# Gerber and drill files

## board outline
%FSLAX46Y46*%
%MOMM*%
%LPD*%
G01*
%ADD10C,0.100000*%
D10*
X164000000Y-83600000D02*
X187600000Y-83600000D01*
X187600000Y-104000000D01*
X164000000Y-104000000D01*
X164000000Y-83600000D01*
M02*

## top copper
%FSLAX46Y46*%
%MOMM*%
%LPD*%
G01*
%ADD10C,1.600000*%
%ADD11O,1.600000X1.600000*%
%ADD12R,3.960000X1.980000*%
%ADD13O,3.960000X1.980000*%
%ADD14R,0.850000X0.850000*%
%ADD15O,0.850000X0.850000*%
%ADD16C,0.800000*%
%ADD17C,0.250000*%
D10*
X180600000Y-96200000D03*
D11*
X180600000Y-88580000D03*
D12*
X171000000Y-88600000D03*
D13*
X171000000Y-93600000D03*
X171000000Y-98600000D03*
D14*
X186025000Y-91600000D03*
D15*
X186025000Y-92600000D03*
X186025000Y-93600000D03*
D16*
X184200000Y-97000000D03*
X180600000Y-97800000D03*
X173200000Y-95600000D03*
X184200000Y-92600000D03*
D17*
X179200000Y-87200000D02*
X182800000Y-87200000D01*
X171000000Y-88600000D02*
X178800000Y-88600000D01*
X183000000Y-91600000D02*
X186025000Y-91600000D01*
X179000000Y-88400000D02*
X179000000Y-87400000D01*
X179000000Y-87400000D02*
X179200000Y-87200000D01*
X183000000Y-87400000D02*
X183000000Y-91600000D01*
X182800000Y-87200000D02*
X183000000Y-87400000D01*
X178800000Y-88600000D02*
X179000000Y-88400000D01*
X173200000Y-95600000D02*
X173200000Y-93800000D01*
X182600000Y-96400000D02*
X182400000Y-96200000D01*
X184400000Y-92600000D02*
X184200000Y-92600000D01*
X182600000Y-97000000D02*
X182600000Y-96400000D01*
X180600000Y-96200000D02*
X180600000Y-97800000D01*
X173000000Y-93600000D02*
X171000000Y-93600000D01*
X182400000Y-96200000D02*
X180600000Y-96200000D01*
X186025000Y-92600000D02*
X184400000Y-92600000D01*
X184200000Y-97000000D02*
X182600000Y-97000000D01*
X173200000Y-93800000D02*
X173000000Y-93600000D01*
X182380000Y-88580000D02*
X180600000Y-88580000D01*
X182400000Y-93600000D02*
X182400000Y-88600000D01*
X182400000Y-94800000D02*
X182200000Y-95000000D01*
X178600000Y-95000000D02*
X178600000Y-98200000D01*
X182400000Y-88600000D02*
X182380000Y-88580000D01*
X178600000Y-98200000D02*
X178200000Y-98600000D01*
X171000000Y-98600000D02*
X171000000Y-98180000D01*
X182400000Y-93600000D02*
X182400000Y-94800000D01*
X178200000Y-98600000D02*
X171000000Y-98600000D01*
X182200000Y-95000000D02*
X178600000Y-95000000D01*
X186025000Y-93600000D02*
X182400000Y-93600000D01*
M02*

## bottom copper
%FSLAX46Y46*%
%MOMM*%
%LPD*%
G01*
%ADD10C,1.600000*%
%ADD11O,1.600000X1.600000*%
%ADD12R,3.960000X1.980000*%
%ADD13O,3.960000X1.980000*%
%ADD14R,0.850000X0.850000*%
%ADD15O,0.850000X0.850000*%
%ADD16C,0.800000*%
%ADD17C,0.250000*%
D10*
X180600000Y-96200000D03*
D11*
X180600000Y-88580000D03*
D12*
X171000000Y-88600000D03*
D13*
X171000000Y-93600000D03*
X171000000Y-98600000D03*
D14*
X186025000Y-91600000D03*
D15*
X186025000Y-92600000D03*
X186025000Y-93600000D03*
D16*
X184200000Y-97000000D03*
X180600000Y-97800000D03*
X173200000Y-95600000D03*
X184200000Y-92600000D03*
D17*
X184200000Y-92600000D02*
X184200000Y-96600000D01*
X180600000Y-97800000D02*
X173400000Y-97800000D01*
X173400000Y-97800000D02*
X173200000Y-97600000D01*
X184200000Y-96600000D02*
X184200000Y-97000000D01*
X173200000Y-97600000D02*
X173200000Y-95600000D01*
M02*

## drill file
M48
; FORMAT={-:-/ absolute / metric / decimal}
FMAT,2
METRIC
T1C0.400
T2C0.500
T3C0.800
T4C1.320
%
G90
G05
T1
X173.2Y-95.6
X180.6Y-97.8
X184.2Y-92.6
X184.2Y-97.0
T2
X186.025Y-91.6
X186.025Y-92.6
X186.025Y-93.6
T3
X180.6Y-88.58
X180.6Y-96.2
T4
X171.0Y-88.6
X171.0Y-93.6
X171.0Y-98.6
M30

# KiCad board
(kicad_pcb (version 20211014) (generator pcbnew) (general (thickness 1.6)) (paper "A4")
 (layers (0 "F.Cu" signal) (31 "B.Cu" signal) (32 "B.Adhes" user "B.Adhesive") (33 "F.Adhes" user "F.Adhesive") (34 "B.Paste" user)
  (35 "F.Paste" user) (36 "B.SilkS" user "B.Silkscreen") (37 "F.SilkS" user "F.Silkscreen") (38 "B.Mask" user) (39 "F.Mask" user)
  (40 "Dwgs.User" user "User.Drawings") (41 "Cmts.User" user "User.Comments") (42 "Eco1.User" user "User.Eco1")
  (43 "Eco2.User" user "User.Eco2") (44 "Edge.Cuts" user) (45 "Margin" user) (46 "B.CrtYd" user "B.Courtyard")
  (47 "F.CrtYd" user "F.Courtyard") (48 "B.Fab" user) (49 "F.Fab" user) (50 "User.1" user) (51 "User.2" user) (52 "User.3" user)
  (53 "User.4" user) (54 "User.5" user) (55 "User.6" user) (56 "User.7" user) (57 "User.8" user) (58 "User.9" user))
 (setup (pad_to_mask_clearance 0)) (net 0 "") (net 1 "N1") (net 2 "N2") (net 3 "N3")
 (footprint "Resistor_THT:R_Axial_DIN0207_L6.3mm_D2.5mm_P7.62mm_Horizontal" (layer "F.Cu") (at 180.6 96.2 90)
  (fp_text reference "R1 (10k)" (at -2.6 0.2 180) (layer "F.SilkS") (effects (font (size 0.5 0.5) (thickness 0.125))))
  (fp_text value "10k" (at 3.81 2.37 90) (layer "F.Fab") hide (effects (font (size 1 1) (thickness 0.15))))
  (pad "1" thru_hole circle (at 0 0 90) (size 1.6 1.6) (drill 0.8) (layers *.Cu *.Mask) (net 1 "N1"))
  (pad "2" thru_hole oval (at 7.62 0 90) (size 1.6 1.6) (drill 0.8) (layers *.Cu *.Mask) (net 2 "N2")))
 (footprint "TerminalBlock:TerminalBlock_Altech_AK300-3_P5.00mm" (layer "F.Cu") (at 171 88.6 -90)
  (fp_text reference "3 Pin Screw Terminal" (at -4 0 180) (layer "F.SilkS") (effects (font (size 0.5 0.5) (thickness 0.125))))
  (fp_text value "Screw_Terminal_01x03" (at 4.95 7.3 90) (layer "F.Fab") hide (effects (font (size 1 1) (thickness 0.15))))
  (pad "1" thru_hole rect (at 0 0 270) (size 1.98 3.96) (drill 1.32) (layers *.Cu *.Mask) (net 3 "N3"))
  (pad "2" thru_hole oval (at 5 0 270) (size 1.98 3.96) (drill 1.32) (layers *.Cu *.Mask) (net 1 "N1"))
  (pad "3" thru_hole oval (at 10 0 270) (size 1.98 3.96) (drill 1.32) (layers *.Cu *.Mask) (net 2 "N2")))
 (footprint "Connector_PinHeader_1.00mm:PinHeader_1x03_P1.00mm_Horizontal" (layer "F.Cu") (at 186.025 91.6)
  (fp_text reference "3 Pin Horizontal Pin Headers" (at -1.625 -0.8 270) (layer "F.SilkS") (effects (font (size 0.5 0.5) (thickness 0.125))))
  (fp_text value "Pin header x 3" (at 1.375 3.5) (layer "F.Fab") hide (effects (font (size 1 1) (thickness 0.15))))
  (pad "1" thru_hole rect (at 0 0) (size 0.85 0.85) (drill 0.5) (layers *.Cu *.Mask) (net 3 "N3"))
  (pad "2" thru_hole oval (at 0 1) (size 0.85 0.85) (drill 0.5) (layers *.Cu *.Mask) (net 1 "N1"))
  (pad "3" thru_hole oval (at 0 2) (size 0.85 0.85) (drill 0.5) (layers *.Cu *.Mask) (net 2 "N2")))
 (gr_rect (start 164 83.6) (end 187.6 104) (layer "Edge.Cuts") (width 0.1) (fill none))
 (segment (start 179.2 87.2) (end 182.8 87.2) (width 0.25) (layer "F.Cu") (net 3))
 (segment (start 171 88.6) (end 178.8 88.6) (width 0.25) (layer "F.Cu") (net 3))
 (segment (start 183 91.6) (end 186.025 91.6) (width 0.25) (layer "F.Cu") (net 3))
 (segment (start 179 88.4) (end 179 87.4) (width 0.25) (layer "F.Cu") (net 3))
 (segment (start 179 87.4) (end 179.2 87.2) (width 0.25) (layer "F.Cu") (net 3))
 (segment (start 183 87.4) (end 183 91.6) (width 0.25) (layer "F.Cu") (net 3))
 (segment (start 182.8 87.2) (end 183 87.4) (width 0.25) (layer "F.Cu") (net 3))
 (segment (start 178.8 88.6) (end 179 88.4) (width 0.25) (layer "F.Cu") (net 3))
 (segment (start 173.2 95.6) (end 173.2 93.8) (width 0.25) (layer "F.Cu") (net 1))
 (segment (start 182.6 96.4) (end 182.4 96.2) (width 0.25) (layer "F.Cu") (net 1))
 (segment (start 184.4 92.6) (end 184.2 92.6) (width 0.25) (layer "F.Cu") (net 1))
 (segment (start 182.6 97) (end 182.6 96.4) (width 0.25) (layer "F.Cu") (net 1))
 (segment (start 180.6 96.2) (end 180.6 97.8) (width 0.25) (layer "F.Cu") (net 1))
 (segment (start 173 93.6) (end 171 93.6) (width 0.25) (layer "F.Cu") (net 1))
 (segment (start 182.4 96.2) (end 180.6 96.2) (width 0.25) (layer "F.Cu") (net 1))
 (segment (start 186.025 92.6) (end 184.4 92.6) (width 0.25) (layer "F.Cu") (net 1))
 (segment (start 184.2 97) (end 182.6 97) (width 0.25) (layer "F.Cu") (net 1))
 (segment (start 173.2 93.8) (end 173 93.6) (width 0.25) (layer "F.Cu") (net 1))
 (via (at 184.2 97) (size 0.8) (drill 0.4) (layers "F.Cu" "B.Cu") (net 1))
 (via (at 180.6 97.8) (size 0.8) (drill 0.4) (layers "F.Cu" "B.Cu") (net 1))
 (via (at 173.2 95.6) (size 0.8) (drill 0.4) (layers "F.Cu" "B.Cu") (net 1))
 (via (at 184.2 92.6) (size 0.8) (drill 0.4) (layers "F.Cu" "B.Cu") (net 1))
 (segment (start 184.2 92.6) (end 184.2 96.6) (width 0.25) (layer "B.Cu") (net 1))
 (segment (start 180.6 97.8) (end 173.4 97.8) (width 0.25) (layer "B.Cu") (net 1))
 (segment (start 173.4 97.8) (end 173.2 97.6) (width 0.25) (layer "B.Cu") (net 1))
 (segment (start 184.2 96.6) (end 184.2 97) (width 0.25) (layer "B.Cu") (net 1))
 (segment (start 173.2 97.6) (end 173.2 95.6) (width 0.25) (layer "B.Cu") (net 1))
 (segment (start 182.38 88.58) (end 180.6 88.58) (width 0.25) (layer "F.Cu") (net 2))
 (segment (start 182.4 93.6) (end 182.4 88.6) (width 0.25) (layer "F.Cu") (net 2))
 (segment (start 182.4 94.8) (end 182.2 95) (width 0.25) (layer "F.Cu") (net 2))
 (segment (start 178.6 95) (end 178.6 98.2) (width 0.25) (layer "F.Cu") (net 2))
 (segment (start 182.4 88.6) (end 182.38 88.58) (width 0.25) (layer "F.Cu") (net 2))
 (segment (start 178.6 98.2) (end 178.2 98.6) (width 0.25) (layer "F.Cu") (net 2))
 (segment (start 171 98.6) (end 171 98.18) (width 0.25) (layer "F.Cu") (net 2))
 (segment (start 182.4 93.6) (end 182.4 94.8) (width 0.25) (layer "F.Cu") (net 2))
 (segment (start 178.2 98.6) (end 171 98.6) (width 0.25) (layer "F.Cu") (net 2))
 (segment (start 182.2 95) (end 178.6 95) (width 0.25) (layer "F.Cu") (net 2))
 (segment (start 186.025 93.6) (end 182.4 93.6) (width 0.25) (layer "F.Cu") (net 2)))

